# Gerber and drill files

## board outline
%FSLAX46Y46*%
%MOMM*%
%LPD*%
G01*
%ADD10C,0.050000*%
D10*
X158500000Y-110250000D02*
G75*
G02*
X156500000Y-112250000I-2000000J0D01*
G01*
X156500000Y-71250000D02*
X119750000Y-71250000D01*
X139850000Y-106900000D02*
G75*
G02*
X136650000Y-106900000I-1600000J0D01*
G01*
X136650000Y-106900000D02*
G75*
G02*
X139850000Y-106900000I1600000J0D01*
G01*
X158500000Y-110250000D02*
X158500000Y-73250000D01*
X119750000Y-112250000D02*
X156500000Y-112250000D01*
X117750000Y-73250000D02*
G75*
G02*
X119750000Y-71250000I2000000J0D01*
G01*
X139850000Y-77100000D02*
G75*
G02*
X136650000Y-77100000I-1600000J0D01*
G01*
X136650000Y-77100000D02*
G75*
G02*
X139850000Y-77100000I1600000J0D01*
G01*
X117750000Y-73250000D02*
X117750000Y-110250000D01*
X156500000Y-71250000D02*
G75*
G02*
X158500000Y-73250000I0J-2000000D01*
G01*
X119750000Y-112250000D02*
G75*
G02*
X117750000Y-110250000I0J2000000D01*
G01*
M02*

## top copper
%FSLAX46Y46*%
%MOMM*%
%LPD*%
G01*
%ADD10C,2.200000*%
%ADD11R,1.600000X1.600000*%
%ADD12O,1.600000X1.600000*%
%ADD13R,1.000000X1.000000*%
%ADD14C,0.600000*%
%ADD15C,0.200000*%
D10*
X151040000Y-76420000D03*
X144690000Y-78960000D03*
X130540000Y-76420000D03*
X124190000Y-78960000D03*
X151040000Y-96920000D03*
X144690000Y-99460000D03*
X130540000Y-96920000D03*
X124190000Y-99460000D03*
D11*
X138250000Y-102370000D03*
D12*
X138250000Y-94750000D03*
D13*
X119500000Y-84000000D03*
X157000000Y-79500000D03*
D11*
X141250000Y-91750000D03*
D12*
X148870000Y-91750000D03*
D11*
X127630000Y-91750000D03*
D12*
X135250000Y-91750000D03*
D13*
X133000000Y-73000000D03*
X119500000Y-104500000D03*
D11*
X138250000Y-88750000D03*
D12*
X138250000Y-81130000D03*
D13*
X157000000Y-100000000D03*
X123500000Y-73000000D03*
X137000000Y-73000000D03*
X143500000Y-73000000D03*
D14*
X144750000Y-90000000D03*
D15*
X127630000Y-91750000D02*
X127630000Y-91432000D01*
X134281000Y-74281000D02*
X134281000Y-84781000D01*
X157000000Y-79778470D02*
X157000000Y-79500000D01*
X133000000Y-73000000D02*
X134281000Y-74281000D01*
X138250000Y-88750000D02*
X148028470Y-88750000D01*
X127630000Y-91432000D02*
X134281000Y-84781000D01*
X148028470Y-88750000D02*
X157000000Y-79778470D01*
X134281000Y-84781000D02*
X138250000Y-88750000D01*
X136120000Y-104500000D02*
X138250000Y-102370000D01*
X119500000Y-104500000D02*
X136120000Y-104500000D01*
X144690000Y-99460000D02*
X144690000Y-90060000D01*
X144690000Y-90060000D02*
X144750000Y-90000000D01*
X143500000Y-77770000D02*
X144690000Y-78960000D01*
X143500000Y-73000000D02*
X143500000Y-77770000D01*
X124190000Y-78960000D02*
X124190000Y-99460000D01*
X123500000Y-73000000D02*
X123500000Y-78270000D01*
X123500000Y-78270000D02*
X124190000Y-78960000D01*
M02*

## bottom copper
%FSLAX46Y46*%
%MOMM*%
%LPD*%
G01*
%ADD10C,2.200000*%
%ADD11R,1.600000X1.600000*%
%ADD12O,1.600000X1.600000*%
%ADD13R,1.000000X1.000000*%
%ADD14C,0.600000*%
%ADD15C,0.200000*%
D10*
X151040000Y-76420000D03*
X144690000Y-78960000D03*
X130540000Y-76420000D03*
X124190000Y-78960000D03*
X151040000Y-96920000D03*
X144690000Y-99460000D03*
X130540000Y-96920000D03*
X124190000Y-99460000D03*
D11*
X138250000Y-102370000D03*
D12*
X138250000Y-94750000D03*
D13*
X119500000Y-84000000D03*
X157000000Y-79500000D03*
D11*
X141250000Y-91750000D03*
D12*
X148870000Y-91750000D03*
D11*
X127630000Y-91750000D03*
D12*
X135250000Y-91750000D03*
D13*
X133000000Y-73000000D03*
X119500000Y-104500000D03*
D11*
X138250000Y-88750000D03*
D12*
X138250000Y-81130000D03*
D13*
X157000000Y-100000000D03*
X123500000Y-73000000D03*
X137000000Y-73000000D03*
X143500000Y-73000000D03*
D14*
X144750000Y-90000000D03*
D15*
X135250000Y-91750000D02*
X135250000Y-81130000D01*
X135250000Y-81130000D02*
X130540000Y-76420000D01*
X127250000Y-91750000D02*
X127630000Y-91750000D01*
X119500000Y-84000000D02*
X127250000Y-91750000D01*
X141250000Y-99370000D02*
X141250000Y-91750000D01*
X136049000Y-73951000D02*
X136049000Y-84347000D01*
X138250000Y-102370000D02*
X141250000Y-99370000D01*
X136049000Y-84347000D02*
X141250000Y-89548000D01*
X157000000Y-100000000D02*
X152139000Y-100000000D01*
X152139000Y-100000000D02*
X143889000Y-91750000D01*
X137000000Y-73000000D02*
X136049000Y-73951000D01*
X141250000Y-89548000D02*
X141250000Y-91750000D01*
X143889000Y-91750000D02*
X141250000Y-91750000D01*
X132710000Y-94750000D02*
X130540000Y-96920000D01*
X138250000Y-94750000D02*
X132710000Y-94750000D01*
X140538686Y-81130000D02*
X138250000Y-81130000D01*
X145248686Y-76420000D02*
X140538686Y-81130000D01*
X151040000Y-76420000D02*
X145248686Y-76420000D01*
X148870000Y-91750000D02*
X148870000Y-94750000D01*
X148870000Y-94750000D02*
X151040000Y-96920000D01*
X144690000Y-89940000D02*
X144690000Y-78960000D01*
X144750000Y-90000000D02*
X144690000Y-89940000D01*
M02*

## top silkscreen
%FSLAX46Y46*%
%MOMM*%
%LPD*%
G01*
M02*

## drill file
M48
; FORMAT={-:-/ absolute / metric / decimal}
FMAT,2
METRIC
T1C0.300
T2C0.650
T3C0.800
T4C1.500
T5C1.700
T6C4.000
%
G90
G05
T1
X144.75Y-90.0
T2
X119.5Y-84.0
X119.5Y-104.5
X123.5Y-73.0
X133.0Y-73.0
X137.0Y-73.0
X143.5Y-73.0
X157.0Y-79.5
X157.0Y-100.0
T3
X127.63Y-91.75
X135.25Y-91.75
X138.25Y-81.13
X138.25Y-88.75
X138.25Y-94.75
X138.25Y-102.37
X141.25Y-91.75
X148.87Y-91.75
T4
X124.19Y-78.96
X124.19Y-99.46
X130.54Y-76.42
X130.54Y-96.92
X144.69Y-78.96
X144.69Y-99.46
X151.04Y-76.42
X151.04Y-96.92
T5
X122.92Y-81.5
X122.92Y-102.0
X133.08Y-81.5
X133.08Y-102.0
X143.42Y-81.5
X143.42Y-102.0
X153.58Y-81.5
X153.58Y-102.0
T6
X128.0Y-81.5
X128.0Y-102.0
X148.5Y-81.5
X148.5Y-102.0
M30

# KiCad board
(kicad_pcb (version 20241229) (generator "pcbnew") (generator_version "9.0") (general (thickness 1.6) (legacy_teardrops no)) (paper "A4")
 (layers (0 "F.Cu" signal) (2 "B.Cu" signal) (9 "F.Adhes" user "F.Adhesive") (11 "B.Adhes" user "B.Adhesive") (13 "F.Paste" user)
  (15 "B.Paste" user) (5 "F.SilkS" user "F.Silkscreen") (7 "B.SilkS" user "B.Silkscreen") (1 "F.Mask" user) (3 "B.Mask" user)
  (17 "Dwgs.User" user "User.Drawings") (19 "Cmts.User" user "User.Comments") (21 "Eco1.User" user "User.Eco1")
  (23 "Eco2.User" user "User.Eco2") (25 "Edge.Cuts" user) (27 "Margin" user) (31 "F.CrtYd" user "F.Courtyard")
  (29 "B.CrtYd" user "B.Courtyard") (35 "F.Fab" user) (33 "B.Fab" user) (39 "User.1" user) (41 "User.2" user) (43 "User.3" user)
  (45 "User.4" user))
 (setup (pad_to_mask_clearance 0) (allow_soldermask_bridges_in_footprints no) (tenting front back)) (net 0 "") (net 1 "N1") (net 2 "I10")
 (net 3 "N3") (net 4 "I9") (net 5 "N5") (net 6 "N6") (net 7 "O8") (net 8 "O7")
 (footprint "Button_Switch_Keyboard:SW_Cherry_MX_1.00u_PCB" (layer "F.Cu") (at 151.04 76.42)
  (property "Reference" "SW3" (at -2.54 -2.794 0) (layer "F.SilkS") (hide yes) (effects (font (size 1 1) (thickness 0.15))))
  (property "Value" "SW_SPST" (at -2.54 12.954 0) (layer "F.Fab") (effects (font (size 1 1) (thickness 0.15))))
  (pad "" np_thru_hole circle (at -7.62 5.08) (size 1.7 1.7) (drill 1.7) (layers "*.Cu" "*.Mask"))
  (pad "" np_thru_hole circle (at -2.54 5.08) (size 4 4) (drill 4) (layers "*.Cu" "*.Mask"))
  (pad "" np_thru_hole circle (at 2.54 5.08) (size 1.7 1.7) (drill 1.7) (layers "*.Cu" "*.Mask"))
  (pad "1" thru_hole circle (at 0 0) (size 2.2 2.2) (drill 1.5) (layers "*.Cu" "*.Mask") (remove_unused_layers no) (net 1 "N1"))
  (pad "2" thru_hole circle (at -6.35 2.54) (size 2.2 2.2) (drill 1.5) (layers "*.Cu" "*.Mask") (remove_unused_layers no) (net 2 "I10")))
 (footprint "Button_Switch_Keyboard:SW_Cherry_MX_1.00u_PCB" (layer "F.Cu") (at 130.54 76.42)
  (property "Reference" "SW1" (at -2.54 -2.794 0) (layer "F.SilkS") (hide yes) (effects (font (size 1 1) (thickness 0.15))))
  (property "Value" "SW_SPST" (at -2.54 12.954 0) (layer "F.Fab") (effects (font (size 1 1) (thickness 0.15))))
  (pad "" np_thru_hole circle (at -7.62 5.08) (size 1.7 1.7) (drill 1.7) (layers "*.Cu" "*.Mask"))
  (pad "" np_thru_hole circle (at -2.54 5.08) (size 4 4) (drill 4) (layers "*.Cu" "*.Mask"))
  (pad "" np_thru_hole circle (at 2.54 5.08) (size 1.7 1.7) (drill 1.7) (layers "*.Cu" "*.Mask"))
  (pad "1" thru_hole circle (at 0 0) (size 2.2 2.2) (drill 1.5) (layers "*.Cu" "*.Mask") (remove_unused_layers no) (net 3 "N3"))
  (pad "2" thru_hole circle (at -6.35 2.54) (size 2.2 2.2) (drill 1.5) (layers "*.Cu" "*.Mask") (remove_unused_layers no) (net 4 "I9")))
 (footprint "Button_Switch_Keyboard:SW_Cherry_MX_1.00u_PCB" (layer "F.Cu") (at 151.04 96.92)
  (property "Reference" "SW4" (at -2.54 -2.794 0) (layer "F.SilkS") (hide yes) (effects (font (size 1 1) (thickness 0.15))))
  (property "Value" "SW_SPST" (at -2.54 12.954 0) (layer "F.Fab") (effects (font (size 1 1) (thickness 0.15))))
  (pad "" np_thru_hole circle (at -7.62 5.08) (size 1.7 1.7) (drill 1.7) (layers "*.Cu" "*.Mask"))
  (pad "" np_thru_hole circle (at -2.54 5.08) (size 4 4) (drill 4) (layers "*.Cu" "*.Mask"))
  (pad "" np_thru_hole circle (at 2.54 5.08) (size 1.7 1.7) (drill 1.7) (layers "*.Cu" "*.Mask"))
  (pad "1" thru_hole circle (at 0 0) (size 2.2 2.2) (drill 1.5) (layers "*.Cu" "*.Mask") (remove_unused_layers no) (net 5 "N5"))
  (pad "2" thru_hole circle (at -6.35 2.54) (size 2.2 2.2) (drill 1.5) (layers "*.Cu" "*.Mask") (remove_unused_layers no) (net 2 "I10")))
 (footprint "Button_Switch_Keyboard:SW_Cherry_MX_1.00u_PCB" (layer "F.Cu") (at 130.54 96.92)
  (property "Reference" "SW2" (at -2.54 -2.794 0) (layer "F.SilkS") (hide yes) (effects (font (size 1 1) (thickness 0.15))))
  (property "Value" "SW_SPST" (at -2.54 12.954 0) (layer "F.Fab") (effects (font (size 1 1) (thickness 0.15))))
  (pad "" np_thru_hole circle (at -7.62 5.08) (size 1.7 1.7) (drill 1.7) (layers "*.Cu" "*.Mask"))
  (pad "" np_thru_hole circle (at -2.54 5.08) (size 4 4) (drill 4) (layers "*.Cu" "*.Mask"))
  (pad "" np_thru_hole circle (at 2.54 5.08) (size 1.7 1.7) (drill 1.7) (layers "*.Cu" "*.Mask"))
  (pad "1" thru_hole circle (at 0 0) (size 2.2 2.2) (drill 1.5) (layers "*.Cu" "*.Mask") (remove_unused_layers no) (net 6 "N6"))
  (pad "2" thru_hole circle (at -6.35 2.54) (size 2.2 2.2) (drill 1.5) (layers "*.Cu" "*.Mask") (remove_unused_layers no) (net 4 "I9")))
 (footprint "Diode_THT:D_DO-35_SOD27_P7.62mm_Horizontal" (layer "B.Cu") (at 138.25 102.37 90)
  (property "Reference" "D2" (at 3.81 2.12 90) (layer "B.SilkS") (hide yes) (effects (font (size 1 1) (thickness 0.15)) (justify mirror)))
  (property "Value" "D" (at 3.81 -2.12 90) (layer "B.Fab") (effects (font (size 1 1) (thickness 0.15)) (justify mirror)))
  (pad "1" thru_hole rect (at 0 0 90) (size 1.6 1.6) (drill 0.8) (layers "*.Cu" "*.Mask") (remove_unused_layers no) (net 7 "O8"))
  (pad "2" thru_hole oval (at 7.62 0 90) (size 1.6 1.6) (drill 0.8) (layers "*.Cu" "*.Mask") (remove_unused_layers no) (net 6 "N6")))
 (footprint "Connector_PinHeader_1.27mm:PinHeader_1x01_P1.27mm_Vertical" (layer "B.Cu") (at 119.5 84)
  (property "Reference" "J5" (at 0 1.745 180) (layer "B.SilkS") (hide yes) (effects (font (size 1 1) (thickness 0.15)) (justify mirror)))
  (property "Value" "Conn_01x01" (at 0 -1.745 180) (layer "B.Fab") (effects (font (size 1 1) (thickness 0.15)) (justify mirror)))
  (pad "1" thru_hole rect (at 0 0) (size 1 1) (drill 0.65) (layers "*.Cu" "*.Mask") (remove_unused_layers no) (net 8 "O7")))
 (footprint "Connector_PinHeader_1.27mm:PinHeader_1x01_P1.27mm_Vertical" (layer "B.Cu") (at 157 79.5)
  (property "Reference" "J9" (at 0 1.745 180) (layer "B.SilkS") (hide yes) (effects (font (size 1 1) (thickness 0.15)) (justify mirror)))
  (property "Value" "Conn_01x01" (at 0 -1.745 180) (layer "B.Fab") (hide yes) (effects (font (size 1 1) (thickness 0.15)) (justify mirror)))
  (pad "1" thru_hole rect (at 0 0) (size 1 1) (drill 0.65) (layers "*.Cu" "*.Mask") (remove_unused_layers no) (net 8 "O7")))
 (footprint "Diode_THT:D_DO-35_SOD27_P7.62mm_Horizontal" (layer "B.Cu") (at 141.25 91.75)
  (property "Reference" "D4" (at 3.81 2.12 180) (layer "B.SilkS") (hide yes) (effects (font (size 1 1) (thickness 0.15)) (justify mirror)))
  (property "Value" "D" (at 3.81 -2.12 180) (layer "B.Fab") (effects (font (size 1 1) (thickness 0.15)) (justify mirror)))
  (pad "1" thru_hole rect (at 0 0) (size 1.6 1.6) (drill 0.8) (layers "*.Cu" "*.Mask") (remove_unused_layers no) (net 7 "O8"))
  (pad "2" thru_hole oval (at 7.62 0) (size 1.6 1.6) (drill 0.8) (layers "*.Cu" "*.Mask") (remove_unused_layers no) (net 5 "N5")))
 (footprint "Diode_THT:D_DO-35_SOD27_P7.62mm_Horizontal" (layer "B.Cu") (at 127.63 91.75)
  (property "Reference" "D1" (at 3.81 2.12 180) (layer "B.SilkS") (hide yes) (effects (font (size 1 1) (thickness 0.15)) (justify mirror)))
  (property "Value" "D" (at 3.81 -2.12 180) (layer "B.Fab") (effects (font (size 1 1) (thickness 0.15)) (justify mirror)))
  (pad "1" thru_hole rect (at 0 0) (size 1.6 1.6) (drill 0.8) (layers "*.Cu" "*.Mask") (remove_unused_layers no) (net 8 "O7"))
  (pad "2" thru_hole oval (at 7.62 0) (size 1.6 1.6) (drill 0.8) (layers "*.Cu" "*.Mask") (remove_unused_layers no) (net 3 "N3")))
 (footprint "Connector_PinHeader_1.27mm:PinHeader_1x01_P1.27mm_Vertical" (layer "B.Cu") (at 133 73)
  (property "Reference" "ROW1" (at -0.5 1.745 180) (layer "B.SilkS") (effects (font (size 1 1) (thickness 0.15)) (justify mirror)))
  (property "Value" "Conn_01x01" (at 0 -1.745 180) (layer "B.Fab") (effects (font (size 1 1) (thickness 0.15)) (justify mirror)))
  (pad "1" thru_hole rect (at 0 0) (size 1 1) (drill 0.65) (layers "*.Cu" "*.Mask") (remove_unused_layers no) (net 8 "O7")))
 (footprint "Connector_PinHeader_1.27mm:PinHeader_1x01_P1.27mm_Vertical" (layer "B.Cu") (at 119.5 104.5)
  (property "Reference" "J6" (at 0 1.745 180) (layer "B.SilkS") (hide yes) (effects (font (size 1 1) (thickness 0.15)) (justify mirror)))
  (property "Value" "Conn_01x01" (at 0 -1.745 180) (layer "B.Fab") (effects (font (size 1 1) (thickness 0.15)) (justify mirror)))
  (pad "1" thru_hole rect (at 0 0) (size 1 1) (drill 0.65) (layers "*.Cu" "*.Mask") (remove_unused_layers no) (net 7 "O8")))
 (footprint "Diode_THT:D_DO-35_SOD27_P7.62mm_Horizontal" (layer "B.Cu") (at 138.25 88.75 90)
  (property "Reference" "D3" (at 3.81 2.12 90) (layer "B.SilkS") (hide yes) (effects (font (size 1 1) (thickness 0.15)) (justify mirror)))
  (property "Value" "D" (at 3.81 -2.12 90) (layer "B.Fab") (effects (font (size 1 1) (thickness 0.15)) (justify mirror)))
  (pad "1" thru_hole rect (at 0 0 90) (size 1.6 1.6) (drill 0.8) (layers "*.Cu" "*.Mask") (remove_unused_layers no) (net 8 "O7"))
  (pad "2" thru_hole oval (at 7.62 0 90) (size 1.6 1.6) (drill 0.8) (layers "*.Cu" "*.Mask") (remove_unused_layers no) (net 1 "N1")))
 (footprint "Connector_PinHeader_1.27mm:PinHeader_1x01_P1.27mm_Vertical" (layer "B.Cu") (at 157 100)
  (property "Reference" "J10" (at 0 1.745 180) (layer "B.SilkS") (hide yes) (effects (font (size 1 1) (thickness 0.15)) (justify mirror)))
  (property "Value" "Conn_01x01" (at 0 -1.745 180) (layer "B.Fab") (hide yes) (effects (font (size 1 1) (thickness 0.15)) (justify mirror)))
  (pad "1" thru_hole rect (at 0 0) (size 1 1) (drill 0.65) (layers "*.Cu" "*.Mask") (remove_unused_layers no) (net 7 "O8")))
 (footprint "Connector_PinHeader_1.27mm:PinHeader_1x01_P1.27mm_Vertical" (layer "B.Cu") (at 123.5 73)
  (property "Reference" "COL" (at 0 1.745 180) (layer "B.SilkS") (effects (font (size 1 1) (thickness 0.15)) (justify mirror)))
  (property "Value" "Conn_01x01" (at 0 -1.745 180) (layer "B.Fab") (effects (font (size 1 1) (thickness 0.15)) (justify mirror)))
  (pad "1" thru_hole rect (at 0 0) (size 1 1) (drill 0.65) (layers "*.Cu" "*.Mask") (remove_unused_layers no) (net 4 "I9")))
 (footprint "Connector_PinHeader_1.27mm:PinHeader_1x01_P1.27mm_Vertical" (layer "B.Cu") (at 137 73)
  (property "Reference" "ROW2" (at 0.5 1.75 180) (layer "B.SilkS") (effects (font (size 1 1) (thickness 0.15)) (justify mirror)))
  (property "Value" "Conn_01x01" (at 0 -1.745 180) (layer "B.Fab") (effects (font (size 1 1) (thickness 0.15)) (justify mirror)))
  (pad "1" thru_hole rect (at 0 0) (size 1 1) (drill 0.65) (layers "*.Cu" "*.Mask") (remove_unused_layers no) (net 7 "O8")))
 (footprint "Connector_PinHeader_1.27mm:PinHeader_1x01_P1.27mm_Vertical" (layer "B.Cu") (at 143.5 73)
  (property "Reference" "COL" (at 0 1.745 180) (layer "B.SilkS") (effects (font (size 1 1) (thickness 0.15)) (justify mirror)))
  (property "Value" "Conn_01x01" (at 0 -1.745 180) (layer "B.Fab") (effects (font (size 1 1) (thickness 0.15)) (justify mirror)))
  (pad "1" thru_hole rect (at 0 0) (size 1 1) (drill 0.65) (layers "*.Cu" "*.Mask") (remove_unused_layers no) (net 2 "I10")))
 (gr_arc (start 158.5 110.25) (mid 157.914214 111.664214) (end 156.5 112.25) (stroke (width 0.05) (type default)) (layer "Edge.Cuts"))
 (gr_line (start 156.5 71.25) (end 119.75 71.25) (stroke (width 0.05) (type default)) (layer "Edge.Cuts"))
 (gr_circle (center 138.25 106.9) (end 139.85 106.9) (stroke (width 0.05) (type solid)) (fill no) (layer "Edge.Cuts"))
 (gr_line (start 158.5 110.25) (end 158.5 73.25) (stroke (width 0.05) (type default)) (layer "Edge.Cuts"))
 (gr_line (start 119.75 112.25) (end 156.5 112.25) (stroke (width 0.05) (type default)) (layer "Edge.Cuts"))
 (gr_arc (start 117.75 73.25) (mid 118.335786 71.835786) (end 119.75 71.25) (stroke (width 0.05) (type default)) (layer "Edge.Cuts"))
 (gr_circle (center 138.25 77.1) (end 139.85 77.1) (stroke (width 0.05) (type solid)) (fill no) (layer "Edge.Cuts"))
 (gr_line (start 117.75 73.25) (end 117.75 110.25) (stroke (width 0.05) (type default)) (layer "Edge.Cuts"))
 (gr_arc (start 156.5 71.25) (mid 157.914214 71.835786) (end 158.5 73.25) (stroke (width 0.05) (type default)) (layer "Edge.Cuts"))
 (gr_arc (start 119.75 112.25) (mid 118.335786 111.664214) (end 117.75 110.25) (stroke (width 0.05) (type default)) (layer "Edge.Cuts"))
 (segment (start 135.25 91.75) (end 135.25 81.13) (width 0.2) (layer "B.Cu") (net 3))
 (segment (start 135.25 81.13) (end 130.54 76.42) (width 0.2) (layer "B.Cu") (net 3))
 (segment (start 127.63 91.75) (end 127.63 91.432) (width 0.2) (layer "F.Cu") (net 8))
 (segment (start 134.281 74.281) (end 134.281 84.781) (width 0.2) (layer "F.Cu") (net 8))
 (segment (start 157 79.77847) (end 157 79.5) (width 0.2) (layer "F.Cu") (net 8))
 (segment (start 133 73) (end 134.281 74.281) (width 0.2) (layer "F.Cu") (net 8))
 (segment (start 138.25 88.75) (end 148.02847 88.75) (width 0.2) (layer "F.Cu") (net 8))
 (segment (start 127.63 91.432) (end 134.281 84.781) (width 0.2) (layer "F.Cu") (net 8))
 (segment (start 148.02847 88.75) (end 157 79.77847) (width 0.2) (layer "F.Cu") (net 8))
 (segment (start 134.281 84.781) (end 138.25 88.75) (width 0.2) (layer "F.Cu") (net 8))
 (segment (start 127.25 91.75) (end 127.63 91.75) (width 0.2) (layer "B.Cu") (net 8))
 (segment (start 119.5 84) (end 127.25 91.75) (width 0.2) (layer "B.Cu") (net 8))
 (segment (start 136.12 104.5) (end 138.25 102.37) (width 0.2) (layer "F.Cu") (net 7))
 (segment (start 119.5 104.5) (end 136.12 104.5) (width 0.2) (layer "F.Cu") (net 7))
 (segment (start 141.25 99.37) (end 141.25 91.75) (width 0.2) (layer "B.Cu") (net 7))
 (segment (start 136.049 73.951) (end 136.049 84.347) (width 0.2) (layer "B.Cu") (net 7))
 (segment (start 138.25 102.37) (end 141.25 99.37) (width 0.2) (layer "B.Cu") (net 7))
 (segment (start 136.049 84.347) (end 141.25 89.548) (width 0.2) (layer "B.Cu") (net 7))
 (segment (start 157 100) (end 152.139 100) (width 0.2) (layer "B.Cu") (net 7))
 (segment (start 152.139 100) (end 143.889 91.75) (width 0.2) (layer "B.Cu") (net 7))
 (segment (start 137 73) (end 136.049 73.951) (width 0.2) (layer "B.Cu") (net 7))
 (segment (start 141.25 89.548) (end 141.25 91.75) (width 0.2) (layer "B.Cu") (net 7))
 (segment (start 143.889 91.75) (end 141.25 91.75) (width 0.2) (layer "B.Cu") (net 7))
 (segment (start 132.71 94.75) (end 130.54 96.92) (width 0.2) (layer "B.Cu") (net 6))
 (segment (start 138.25 94.75) (end 132.71 94.75) (width 0.2) (layer "B.Cu") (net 6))
 (segment (start 140.538686 81.13) (end 138.25 81.13) (width 0.2) (layer "B.Cu") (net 1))
 (segment (start 145.248686 76.42) (end 140.538686 81.13) (width 0.2) (layer "B.Cu") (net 1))
 (segment (start 151.04 76.42) (end 145.248686 76.42) (width 0.2) (layer "B.Cu") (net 1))
 (segment (start 148.87 91.75) (end 148.87 94.75) (width 0.2) (layer "B.Cu") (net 5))
 (segment (start 148.87 94.75) (end 151.04 96.92) (width 0.2) (layer "B.Cu") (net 5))
 (segment (start 144.69 99.46) (end 144.69 90.06) (width 0.2) (layer "F.Cu") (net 2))
 (segment (start 144.69 90.06) (end 144.75 90) (width 0.2) (layer "F.Cu") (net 2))
 (segment (start 143.5 77.77) (end 144.69 78.96) (width 0.2) (layer "F.Cu") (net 2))
 (segment (start 143.5 73) (end 143.5 77.77) (width 0.2) (layer "F.Cu") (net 2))
 (via (at 144.75 90) (size 0.6) (drill 0.3) (layers "F.Cu" "B.Cu") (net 2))
 (segment (start 144.69 89.94) (end 144.69 78.96) (width 0.2) (layer "B.Cu") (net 2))
 (segment (start 144.75 90) (end 144.69 89.94) (width 0.2) (layer "B.Cu") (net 2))
 (segment (start 124.19 78.96) (end 124.19 99.46) (width 0.2) (layer "F.Cu") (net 4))
 (segment (start 123.5 73) (end 123.5 78.27) (width 0.2) (layer "F.Cu") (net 4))
 (segment (start 123.5 78.27) (end 124.19 78.96) (width 0.2) (layer "F.Cu") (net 4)))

